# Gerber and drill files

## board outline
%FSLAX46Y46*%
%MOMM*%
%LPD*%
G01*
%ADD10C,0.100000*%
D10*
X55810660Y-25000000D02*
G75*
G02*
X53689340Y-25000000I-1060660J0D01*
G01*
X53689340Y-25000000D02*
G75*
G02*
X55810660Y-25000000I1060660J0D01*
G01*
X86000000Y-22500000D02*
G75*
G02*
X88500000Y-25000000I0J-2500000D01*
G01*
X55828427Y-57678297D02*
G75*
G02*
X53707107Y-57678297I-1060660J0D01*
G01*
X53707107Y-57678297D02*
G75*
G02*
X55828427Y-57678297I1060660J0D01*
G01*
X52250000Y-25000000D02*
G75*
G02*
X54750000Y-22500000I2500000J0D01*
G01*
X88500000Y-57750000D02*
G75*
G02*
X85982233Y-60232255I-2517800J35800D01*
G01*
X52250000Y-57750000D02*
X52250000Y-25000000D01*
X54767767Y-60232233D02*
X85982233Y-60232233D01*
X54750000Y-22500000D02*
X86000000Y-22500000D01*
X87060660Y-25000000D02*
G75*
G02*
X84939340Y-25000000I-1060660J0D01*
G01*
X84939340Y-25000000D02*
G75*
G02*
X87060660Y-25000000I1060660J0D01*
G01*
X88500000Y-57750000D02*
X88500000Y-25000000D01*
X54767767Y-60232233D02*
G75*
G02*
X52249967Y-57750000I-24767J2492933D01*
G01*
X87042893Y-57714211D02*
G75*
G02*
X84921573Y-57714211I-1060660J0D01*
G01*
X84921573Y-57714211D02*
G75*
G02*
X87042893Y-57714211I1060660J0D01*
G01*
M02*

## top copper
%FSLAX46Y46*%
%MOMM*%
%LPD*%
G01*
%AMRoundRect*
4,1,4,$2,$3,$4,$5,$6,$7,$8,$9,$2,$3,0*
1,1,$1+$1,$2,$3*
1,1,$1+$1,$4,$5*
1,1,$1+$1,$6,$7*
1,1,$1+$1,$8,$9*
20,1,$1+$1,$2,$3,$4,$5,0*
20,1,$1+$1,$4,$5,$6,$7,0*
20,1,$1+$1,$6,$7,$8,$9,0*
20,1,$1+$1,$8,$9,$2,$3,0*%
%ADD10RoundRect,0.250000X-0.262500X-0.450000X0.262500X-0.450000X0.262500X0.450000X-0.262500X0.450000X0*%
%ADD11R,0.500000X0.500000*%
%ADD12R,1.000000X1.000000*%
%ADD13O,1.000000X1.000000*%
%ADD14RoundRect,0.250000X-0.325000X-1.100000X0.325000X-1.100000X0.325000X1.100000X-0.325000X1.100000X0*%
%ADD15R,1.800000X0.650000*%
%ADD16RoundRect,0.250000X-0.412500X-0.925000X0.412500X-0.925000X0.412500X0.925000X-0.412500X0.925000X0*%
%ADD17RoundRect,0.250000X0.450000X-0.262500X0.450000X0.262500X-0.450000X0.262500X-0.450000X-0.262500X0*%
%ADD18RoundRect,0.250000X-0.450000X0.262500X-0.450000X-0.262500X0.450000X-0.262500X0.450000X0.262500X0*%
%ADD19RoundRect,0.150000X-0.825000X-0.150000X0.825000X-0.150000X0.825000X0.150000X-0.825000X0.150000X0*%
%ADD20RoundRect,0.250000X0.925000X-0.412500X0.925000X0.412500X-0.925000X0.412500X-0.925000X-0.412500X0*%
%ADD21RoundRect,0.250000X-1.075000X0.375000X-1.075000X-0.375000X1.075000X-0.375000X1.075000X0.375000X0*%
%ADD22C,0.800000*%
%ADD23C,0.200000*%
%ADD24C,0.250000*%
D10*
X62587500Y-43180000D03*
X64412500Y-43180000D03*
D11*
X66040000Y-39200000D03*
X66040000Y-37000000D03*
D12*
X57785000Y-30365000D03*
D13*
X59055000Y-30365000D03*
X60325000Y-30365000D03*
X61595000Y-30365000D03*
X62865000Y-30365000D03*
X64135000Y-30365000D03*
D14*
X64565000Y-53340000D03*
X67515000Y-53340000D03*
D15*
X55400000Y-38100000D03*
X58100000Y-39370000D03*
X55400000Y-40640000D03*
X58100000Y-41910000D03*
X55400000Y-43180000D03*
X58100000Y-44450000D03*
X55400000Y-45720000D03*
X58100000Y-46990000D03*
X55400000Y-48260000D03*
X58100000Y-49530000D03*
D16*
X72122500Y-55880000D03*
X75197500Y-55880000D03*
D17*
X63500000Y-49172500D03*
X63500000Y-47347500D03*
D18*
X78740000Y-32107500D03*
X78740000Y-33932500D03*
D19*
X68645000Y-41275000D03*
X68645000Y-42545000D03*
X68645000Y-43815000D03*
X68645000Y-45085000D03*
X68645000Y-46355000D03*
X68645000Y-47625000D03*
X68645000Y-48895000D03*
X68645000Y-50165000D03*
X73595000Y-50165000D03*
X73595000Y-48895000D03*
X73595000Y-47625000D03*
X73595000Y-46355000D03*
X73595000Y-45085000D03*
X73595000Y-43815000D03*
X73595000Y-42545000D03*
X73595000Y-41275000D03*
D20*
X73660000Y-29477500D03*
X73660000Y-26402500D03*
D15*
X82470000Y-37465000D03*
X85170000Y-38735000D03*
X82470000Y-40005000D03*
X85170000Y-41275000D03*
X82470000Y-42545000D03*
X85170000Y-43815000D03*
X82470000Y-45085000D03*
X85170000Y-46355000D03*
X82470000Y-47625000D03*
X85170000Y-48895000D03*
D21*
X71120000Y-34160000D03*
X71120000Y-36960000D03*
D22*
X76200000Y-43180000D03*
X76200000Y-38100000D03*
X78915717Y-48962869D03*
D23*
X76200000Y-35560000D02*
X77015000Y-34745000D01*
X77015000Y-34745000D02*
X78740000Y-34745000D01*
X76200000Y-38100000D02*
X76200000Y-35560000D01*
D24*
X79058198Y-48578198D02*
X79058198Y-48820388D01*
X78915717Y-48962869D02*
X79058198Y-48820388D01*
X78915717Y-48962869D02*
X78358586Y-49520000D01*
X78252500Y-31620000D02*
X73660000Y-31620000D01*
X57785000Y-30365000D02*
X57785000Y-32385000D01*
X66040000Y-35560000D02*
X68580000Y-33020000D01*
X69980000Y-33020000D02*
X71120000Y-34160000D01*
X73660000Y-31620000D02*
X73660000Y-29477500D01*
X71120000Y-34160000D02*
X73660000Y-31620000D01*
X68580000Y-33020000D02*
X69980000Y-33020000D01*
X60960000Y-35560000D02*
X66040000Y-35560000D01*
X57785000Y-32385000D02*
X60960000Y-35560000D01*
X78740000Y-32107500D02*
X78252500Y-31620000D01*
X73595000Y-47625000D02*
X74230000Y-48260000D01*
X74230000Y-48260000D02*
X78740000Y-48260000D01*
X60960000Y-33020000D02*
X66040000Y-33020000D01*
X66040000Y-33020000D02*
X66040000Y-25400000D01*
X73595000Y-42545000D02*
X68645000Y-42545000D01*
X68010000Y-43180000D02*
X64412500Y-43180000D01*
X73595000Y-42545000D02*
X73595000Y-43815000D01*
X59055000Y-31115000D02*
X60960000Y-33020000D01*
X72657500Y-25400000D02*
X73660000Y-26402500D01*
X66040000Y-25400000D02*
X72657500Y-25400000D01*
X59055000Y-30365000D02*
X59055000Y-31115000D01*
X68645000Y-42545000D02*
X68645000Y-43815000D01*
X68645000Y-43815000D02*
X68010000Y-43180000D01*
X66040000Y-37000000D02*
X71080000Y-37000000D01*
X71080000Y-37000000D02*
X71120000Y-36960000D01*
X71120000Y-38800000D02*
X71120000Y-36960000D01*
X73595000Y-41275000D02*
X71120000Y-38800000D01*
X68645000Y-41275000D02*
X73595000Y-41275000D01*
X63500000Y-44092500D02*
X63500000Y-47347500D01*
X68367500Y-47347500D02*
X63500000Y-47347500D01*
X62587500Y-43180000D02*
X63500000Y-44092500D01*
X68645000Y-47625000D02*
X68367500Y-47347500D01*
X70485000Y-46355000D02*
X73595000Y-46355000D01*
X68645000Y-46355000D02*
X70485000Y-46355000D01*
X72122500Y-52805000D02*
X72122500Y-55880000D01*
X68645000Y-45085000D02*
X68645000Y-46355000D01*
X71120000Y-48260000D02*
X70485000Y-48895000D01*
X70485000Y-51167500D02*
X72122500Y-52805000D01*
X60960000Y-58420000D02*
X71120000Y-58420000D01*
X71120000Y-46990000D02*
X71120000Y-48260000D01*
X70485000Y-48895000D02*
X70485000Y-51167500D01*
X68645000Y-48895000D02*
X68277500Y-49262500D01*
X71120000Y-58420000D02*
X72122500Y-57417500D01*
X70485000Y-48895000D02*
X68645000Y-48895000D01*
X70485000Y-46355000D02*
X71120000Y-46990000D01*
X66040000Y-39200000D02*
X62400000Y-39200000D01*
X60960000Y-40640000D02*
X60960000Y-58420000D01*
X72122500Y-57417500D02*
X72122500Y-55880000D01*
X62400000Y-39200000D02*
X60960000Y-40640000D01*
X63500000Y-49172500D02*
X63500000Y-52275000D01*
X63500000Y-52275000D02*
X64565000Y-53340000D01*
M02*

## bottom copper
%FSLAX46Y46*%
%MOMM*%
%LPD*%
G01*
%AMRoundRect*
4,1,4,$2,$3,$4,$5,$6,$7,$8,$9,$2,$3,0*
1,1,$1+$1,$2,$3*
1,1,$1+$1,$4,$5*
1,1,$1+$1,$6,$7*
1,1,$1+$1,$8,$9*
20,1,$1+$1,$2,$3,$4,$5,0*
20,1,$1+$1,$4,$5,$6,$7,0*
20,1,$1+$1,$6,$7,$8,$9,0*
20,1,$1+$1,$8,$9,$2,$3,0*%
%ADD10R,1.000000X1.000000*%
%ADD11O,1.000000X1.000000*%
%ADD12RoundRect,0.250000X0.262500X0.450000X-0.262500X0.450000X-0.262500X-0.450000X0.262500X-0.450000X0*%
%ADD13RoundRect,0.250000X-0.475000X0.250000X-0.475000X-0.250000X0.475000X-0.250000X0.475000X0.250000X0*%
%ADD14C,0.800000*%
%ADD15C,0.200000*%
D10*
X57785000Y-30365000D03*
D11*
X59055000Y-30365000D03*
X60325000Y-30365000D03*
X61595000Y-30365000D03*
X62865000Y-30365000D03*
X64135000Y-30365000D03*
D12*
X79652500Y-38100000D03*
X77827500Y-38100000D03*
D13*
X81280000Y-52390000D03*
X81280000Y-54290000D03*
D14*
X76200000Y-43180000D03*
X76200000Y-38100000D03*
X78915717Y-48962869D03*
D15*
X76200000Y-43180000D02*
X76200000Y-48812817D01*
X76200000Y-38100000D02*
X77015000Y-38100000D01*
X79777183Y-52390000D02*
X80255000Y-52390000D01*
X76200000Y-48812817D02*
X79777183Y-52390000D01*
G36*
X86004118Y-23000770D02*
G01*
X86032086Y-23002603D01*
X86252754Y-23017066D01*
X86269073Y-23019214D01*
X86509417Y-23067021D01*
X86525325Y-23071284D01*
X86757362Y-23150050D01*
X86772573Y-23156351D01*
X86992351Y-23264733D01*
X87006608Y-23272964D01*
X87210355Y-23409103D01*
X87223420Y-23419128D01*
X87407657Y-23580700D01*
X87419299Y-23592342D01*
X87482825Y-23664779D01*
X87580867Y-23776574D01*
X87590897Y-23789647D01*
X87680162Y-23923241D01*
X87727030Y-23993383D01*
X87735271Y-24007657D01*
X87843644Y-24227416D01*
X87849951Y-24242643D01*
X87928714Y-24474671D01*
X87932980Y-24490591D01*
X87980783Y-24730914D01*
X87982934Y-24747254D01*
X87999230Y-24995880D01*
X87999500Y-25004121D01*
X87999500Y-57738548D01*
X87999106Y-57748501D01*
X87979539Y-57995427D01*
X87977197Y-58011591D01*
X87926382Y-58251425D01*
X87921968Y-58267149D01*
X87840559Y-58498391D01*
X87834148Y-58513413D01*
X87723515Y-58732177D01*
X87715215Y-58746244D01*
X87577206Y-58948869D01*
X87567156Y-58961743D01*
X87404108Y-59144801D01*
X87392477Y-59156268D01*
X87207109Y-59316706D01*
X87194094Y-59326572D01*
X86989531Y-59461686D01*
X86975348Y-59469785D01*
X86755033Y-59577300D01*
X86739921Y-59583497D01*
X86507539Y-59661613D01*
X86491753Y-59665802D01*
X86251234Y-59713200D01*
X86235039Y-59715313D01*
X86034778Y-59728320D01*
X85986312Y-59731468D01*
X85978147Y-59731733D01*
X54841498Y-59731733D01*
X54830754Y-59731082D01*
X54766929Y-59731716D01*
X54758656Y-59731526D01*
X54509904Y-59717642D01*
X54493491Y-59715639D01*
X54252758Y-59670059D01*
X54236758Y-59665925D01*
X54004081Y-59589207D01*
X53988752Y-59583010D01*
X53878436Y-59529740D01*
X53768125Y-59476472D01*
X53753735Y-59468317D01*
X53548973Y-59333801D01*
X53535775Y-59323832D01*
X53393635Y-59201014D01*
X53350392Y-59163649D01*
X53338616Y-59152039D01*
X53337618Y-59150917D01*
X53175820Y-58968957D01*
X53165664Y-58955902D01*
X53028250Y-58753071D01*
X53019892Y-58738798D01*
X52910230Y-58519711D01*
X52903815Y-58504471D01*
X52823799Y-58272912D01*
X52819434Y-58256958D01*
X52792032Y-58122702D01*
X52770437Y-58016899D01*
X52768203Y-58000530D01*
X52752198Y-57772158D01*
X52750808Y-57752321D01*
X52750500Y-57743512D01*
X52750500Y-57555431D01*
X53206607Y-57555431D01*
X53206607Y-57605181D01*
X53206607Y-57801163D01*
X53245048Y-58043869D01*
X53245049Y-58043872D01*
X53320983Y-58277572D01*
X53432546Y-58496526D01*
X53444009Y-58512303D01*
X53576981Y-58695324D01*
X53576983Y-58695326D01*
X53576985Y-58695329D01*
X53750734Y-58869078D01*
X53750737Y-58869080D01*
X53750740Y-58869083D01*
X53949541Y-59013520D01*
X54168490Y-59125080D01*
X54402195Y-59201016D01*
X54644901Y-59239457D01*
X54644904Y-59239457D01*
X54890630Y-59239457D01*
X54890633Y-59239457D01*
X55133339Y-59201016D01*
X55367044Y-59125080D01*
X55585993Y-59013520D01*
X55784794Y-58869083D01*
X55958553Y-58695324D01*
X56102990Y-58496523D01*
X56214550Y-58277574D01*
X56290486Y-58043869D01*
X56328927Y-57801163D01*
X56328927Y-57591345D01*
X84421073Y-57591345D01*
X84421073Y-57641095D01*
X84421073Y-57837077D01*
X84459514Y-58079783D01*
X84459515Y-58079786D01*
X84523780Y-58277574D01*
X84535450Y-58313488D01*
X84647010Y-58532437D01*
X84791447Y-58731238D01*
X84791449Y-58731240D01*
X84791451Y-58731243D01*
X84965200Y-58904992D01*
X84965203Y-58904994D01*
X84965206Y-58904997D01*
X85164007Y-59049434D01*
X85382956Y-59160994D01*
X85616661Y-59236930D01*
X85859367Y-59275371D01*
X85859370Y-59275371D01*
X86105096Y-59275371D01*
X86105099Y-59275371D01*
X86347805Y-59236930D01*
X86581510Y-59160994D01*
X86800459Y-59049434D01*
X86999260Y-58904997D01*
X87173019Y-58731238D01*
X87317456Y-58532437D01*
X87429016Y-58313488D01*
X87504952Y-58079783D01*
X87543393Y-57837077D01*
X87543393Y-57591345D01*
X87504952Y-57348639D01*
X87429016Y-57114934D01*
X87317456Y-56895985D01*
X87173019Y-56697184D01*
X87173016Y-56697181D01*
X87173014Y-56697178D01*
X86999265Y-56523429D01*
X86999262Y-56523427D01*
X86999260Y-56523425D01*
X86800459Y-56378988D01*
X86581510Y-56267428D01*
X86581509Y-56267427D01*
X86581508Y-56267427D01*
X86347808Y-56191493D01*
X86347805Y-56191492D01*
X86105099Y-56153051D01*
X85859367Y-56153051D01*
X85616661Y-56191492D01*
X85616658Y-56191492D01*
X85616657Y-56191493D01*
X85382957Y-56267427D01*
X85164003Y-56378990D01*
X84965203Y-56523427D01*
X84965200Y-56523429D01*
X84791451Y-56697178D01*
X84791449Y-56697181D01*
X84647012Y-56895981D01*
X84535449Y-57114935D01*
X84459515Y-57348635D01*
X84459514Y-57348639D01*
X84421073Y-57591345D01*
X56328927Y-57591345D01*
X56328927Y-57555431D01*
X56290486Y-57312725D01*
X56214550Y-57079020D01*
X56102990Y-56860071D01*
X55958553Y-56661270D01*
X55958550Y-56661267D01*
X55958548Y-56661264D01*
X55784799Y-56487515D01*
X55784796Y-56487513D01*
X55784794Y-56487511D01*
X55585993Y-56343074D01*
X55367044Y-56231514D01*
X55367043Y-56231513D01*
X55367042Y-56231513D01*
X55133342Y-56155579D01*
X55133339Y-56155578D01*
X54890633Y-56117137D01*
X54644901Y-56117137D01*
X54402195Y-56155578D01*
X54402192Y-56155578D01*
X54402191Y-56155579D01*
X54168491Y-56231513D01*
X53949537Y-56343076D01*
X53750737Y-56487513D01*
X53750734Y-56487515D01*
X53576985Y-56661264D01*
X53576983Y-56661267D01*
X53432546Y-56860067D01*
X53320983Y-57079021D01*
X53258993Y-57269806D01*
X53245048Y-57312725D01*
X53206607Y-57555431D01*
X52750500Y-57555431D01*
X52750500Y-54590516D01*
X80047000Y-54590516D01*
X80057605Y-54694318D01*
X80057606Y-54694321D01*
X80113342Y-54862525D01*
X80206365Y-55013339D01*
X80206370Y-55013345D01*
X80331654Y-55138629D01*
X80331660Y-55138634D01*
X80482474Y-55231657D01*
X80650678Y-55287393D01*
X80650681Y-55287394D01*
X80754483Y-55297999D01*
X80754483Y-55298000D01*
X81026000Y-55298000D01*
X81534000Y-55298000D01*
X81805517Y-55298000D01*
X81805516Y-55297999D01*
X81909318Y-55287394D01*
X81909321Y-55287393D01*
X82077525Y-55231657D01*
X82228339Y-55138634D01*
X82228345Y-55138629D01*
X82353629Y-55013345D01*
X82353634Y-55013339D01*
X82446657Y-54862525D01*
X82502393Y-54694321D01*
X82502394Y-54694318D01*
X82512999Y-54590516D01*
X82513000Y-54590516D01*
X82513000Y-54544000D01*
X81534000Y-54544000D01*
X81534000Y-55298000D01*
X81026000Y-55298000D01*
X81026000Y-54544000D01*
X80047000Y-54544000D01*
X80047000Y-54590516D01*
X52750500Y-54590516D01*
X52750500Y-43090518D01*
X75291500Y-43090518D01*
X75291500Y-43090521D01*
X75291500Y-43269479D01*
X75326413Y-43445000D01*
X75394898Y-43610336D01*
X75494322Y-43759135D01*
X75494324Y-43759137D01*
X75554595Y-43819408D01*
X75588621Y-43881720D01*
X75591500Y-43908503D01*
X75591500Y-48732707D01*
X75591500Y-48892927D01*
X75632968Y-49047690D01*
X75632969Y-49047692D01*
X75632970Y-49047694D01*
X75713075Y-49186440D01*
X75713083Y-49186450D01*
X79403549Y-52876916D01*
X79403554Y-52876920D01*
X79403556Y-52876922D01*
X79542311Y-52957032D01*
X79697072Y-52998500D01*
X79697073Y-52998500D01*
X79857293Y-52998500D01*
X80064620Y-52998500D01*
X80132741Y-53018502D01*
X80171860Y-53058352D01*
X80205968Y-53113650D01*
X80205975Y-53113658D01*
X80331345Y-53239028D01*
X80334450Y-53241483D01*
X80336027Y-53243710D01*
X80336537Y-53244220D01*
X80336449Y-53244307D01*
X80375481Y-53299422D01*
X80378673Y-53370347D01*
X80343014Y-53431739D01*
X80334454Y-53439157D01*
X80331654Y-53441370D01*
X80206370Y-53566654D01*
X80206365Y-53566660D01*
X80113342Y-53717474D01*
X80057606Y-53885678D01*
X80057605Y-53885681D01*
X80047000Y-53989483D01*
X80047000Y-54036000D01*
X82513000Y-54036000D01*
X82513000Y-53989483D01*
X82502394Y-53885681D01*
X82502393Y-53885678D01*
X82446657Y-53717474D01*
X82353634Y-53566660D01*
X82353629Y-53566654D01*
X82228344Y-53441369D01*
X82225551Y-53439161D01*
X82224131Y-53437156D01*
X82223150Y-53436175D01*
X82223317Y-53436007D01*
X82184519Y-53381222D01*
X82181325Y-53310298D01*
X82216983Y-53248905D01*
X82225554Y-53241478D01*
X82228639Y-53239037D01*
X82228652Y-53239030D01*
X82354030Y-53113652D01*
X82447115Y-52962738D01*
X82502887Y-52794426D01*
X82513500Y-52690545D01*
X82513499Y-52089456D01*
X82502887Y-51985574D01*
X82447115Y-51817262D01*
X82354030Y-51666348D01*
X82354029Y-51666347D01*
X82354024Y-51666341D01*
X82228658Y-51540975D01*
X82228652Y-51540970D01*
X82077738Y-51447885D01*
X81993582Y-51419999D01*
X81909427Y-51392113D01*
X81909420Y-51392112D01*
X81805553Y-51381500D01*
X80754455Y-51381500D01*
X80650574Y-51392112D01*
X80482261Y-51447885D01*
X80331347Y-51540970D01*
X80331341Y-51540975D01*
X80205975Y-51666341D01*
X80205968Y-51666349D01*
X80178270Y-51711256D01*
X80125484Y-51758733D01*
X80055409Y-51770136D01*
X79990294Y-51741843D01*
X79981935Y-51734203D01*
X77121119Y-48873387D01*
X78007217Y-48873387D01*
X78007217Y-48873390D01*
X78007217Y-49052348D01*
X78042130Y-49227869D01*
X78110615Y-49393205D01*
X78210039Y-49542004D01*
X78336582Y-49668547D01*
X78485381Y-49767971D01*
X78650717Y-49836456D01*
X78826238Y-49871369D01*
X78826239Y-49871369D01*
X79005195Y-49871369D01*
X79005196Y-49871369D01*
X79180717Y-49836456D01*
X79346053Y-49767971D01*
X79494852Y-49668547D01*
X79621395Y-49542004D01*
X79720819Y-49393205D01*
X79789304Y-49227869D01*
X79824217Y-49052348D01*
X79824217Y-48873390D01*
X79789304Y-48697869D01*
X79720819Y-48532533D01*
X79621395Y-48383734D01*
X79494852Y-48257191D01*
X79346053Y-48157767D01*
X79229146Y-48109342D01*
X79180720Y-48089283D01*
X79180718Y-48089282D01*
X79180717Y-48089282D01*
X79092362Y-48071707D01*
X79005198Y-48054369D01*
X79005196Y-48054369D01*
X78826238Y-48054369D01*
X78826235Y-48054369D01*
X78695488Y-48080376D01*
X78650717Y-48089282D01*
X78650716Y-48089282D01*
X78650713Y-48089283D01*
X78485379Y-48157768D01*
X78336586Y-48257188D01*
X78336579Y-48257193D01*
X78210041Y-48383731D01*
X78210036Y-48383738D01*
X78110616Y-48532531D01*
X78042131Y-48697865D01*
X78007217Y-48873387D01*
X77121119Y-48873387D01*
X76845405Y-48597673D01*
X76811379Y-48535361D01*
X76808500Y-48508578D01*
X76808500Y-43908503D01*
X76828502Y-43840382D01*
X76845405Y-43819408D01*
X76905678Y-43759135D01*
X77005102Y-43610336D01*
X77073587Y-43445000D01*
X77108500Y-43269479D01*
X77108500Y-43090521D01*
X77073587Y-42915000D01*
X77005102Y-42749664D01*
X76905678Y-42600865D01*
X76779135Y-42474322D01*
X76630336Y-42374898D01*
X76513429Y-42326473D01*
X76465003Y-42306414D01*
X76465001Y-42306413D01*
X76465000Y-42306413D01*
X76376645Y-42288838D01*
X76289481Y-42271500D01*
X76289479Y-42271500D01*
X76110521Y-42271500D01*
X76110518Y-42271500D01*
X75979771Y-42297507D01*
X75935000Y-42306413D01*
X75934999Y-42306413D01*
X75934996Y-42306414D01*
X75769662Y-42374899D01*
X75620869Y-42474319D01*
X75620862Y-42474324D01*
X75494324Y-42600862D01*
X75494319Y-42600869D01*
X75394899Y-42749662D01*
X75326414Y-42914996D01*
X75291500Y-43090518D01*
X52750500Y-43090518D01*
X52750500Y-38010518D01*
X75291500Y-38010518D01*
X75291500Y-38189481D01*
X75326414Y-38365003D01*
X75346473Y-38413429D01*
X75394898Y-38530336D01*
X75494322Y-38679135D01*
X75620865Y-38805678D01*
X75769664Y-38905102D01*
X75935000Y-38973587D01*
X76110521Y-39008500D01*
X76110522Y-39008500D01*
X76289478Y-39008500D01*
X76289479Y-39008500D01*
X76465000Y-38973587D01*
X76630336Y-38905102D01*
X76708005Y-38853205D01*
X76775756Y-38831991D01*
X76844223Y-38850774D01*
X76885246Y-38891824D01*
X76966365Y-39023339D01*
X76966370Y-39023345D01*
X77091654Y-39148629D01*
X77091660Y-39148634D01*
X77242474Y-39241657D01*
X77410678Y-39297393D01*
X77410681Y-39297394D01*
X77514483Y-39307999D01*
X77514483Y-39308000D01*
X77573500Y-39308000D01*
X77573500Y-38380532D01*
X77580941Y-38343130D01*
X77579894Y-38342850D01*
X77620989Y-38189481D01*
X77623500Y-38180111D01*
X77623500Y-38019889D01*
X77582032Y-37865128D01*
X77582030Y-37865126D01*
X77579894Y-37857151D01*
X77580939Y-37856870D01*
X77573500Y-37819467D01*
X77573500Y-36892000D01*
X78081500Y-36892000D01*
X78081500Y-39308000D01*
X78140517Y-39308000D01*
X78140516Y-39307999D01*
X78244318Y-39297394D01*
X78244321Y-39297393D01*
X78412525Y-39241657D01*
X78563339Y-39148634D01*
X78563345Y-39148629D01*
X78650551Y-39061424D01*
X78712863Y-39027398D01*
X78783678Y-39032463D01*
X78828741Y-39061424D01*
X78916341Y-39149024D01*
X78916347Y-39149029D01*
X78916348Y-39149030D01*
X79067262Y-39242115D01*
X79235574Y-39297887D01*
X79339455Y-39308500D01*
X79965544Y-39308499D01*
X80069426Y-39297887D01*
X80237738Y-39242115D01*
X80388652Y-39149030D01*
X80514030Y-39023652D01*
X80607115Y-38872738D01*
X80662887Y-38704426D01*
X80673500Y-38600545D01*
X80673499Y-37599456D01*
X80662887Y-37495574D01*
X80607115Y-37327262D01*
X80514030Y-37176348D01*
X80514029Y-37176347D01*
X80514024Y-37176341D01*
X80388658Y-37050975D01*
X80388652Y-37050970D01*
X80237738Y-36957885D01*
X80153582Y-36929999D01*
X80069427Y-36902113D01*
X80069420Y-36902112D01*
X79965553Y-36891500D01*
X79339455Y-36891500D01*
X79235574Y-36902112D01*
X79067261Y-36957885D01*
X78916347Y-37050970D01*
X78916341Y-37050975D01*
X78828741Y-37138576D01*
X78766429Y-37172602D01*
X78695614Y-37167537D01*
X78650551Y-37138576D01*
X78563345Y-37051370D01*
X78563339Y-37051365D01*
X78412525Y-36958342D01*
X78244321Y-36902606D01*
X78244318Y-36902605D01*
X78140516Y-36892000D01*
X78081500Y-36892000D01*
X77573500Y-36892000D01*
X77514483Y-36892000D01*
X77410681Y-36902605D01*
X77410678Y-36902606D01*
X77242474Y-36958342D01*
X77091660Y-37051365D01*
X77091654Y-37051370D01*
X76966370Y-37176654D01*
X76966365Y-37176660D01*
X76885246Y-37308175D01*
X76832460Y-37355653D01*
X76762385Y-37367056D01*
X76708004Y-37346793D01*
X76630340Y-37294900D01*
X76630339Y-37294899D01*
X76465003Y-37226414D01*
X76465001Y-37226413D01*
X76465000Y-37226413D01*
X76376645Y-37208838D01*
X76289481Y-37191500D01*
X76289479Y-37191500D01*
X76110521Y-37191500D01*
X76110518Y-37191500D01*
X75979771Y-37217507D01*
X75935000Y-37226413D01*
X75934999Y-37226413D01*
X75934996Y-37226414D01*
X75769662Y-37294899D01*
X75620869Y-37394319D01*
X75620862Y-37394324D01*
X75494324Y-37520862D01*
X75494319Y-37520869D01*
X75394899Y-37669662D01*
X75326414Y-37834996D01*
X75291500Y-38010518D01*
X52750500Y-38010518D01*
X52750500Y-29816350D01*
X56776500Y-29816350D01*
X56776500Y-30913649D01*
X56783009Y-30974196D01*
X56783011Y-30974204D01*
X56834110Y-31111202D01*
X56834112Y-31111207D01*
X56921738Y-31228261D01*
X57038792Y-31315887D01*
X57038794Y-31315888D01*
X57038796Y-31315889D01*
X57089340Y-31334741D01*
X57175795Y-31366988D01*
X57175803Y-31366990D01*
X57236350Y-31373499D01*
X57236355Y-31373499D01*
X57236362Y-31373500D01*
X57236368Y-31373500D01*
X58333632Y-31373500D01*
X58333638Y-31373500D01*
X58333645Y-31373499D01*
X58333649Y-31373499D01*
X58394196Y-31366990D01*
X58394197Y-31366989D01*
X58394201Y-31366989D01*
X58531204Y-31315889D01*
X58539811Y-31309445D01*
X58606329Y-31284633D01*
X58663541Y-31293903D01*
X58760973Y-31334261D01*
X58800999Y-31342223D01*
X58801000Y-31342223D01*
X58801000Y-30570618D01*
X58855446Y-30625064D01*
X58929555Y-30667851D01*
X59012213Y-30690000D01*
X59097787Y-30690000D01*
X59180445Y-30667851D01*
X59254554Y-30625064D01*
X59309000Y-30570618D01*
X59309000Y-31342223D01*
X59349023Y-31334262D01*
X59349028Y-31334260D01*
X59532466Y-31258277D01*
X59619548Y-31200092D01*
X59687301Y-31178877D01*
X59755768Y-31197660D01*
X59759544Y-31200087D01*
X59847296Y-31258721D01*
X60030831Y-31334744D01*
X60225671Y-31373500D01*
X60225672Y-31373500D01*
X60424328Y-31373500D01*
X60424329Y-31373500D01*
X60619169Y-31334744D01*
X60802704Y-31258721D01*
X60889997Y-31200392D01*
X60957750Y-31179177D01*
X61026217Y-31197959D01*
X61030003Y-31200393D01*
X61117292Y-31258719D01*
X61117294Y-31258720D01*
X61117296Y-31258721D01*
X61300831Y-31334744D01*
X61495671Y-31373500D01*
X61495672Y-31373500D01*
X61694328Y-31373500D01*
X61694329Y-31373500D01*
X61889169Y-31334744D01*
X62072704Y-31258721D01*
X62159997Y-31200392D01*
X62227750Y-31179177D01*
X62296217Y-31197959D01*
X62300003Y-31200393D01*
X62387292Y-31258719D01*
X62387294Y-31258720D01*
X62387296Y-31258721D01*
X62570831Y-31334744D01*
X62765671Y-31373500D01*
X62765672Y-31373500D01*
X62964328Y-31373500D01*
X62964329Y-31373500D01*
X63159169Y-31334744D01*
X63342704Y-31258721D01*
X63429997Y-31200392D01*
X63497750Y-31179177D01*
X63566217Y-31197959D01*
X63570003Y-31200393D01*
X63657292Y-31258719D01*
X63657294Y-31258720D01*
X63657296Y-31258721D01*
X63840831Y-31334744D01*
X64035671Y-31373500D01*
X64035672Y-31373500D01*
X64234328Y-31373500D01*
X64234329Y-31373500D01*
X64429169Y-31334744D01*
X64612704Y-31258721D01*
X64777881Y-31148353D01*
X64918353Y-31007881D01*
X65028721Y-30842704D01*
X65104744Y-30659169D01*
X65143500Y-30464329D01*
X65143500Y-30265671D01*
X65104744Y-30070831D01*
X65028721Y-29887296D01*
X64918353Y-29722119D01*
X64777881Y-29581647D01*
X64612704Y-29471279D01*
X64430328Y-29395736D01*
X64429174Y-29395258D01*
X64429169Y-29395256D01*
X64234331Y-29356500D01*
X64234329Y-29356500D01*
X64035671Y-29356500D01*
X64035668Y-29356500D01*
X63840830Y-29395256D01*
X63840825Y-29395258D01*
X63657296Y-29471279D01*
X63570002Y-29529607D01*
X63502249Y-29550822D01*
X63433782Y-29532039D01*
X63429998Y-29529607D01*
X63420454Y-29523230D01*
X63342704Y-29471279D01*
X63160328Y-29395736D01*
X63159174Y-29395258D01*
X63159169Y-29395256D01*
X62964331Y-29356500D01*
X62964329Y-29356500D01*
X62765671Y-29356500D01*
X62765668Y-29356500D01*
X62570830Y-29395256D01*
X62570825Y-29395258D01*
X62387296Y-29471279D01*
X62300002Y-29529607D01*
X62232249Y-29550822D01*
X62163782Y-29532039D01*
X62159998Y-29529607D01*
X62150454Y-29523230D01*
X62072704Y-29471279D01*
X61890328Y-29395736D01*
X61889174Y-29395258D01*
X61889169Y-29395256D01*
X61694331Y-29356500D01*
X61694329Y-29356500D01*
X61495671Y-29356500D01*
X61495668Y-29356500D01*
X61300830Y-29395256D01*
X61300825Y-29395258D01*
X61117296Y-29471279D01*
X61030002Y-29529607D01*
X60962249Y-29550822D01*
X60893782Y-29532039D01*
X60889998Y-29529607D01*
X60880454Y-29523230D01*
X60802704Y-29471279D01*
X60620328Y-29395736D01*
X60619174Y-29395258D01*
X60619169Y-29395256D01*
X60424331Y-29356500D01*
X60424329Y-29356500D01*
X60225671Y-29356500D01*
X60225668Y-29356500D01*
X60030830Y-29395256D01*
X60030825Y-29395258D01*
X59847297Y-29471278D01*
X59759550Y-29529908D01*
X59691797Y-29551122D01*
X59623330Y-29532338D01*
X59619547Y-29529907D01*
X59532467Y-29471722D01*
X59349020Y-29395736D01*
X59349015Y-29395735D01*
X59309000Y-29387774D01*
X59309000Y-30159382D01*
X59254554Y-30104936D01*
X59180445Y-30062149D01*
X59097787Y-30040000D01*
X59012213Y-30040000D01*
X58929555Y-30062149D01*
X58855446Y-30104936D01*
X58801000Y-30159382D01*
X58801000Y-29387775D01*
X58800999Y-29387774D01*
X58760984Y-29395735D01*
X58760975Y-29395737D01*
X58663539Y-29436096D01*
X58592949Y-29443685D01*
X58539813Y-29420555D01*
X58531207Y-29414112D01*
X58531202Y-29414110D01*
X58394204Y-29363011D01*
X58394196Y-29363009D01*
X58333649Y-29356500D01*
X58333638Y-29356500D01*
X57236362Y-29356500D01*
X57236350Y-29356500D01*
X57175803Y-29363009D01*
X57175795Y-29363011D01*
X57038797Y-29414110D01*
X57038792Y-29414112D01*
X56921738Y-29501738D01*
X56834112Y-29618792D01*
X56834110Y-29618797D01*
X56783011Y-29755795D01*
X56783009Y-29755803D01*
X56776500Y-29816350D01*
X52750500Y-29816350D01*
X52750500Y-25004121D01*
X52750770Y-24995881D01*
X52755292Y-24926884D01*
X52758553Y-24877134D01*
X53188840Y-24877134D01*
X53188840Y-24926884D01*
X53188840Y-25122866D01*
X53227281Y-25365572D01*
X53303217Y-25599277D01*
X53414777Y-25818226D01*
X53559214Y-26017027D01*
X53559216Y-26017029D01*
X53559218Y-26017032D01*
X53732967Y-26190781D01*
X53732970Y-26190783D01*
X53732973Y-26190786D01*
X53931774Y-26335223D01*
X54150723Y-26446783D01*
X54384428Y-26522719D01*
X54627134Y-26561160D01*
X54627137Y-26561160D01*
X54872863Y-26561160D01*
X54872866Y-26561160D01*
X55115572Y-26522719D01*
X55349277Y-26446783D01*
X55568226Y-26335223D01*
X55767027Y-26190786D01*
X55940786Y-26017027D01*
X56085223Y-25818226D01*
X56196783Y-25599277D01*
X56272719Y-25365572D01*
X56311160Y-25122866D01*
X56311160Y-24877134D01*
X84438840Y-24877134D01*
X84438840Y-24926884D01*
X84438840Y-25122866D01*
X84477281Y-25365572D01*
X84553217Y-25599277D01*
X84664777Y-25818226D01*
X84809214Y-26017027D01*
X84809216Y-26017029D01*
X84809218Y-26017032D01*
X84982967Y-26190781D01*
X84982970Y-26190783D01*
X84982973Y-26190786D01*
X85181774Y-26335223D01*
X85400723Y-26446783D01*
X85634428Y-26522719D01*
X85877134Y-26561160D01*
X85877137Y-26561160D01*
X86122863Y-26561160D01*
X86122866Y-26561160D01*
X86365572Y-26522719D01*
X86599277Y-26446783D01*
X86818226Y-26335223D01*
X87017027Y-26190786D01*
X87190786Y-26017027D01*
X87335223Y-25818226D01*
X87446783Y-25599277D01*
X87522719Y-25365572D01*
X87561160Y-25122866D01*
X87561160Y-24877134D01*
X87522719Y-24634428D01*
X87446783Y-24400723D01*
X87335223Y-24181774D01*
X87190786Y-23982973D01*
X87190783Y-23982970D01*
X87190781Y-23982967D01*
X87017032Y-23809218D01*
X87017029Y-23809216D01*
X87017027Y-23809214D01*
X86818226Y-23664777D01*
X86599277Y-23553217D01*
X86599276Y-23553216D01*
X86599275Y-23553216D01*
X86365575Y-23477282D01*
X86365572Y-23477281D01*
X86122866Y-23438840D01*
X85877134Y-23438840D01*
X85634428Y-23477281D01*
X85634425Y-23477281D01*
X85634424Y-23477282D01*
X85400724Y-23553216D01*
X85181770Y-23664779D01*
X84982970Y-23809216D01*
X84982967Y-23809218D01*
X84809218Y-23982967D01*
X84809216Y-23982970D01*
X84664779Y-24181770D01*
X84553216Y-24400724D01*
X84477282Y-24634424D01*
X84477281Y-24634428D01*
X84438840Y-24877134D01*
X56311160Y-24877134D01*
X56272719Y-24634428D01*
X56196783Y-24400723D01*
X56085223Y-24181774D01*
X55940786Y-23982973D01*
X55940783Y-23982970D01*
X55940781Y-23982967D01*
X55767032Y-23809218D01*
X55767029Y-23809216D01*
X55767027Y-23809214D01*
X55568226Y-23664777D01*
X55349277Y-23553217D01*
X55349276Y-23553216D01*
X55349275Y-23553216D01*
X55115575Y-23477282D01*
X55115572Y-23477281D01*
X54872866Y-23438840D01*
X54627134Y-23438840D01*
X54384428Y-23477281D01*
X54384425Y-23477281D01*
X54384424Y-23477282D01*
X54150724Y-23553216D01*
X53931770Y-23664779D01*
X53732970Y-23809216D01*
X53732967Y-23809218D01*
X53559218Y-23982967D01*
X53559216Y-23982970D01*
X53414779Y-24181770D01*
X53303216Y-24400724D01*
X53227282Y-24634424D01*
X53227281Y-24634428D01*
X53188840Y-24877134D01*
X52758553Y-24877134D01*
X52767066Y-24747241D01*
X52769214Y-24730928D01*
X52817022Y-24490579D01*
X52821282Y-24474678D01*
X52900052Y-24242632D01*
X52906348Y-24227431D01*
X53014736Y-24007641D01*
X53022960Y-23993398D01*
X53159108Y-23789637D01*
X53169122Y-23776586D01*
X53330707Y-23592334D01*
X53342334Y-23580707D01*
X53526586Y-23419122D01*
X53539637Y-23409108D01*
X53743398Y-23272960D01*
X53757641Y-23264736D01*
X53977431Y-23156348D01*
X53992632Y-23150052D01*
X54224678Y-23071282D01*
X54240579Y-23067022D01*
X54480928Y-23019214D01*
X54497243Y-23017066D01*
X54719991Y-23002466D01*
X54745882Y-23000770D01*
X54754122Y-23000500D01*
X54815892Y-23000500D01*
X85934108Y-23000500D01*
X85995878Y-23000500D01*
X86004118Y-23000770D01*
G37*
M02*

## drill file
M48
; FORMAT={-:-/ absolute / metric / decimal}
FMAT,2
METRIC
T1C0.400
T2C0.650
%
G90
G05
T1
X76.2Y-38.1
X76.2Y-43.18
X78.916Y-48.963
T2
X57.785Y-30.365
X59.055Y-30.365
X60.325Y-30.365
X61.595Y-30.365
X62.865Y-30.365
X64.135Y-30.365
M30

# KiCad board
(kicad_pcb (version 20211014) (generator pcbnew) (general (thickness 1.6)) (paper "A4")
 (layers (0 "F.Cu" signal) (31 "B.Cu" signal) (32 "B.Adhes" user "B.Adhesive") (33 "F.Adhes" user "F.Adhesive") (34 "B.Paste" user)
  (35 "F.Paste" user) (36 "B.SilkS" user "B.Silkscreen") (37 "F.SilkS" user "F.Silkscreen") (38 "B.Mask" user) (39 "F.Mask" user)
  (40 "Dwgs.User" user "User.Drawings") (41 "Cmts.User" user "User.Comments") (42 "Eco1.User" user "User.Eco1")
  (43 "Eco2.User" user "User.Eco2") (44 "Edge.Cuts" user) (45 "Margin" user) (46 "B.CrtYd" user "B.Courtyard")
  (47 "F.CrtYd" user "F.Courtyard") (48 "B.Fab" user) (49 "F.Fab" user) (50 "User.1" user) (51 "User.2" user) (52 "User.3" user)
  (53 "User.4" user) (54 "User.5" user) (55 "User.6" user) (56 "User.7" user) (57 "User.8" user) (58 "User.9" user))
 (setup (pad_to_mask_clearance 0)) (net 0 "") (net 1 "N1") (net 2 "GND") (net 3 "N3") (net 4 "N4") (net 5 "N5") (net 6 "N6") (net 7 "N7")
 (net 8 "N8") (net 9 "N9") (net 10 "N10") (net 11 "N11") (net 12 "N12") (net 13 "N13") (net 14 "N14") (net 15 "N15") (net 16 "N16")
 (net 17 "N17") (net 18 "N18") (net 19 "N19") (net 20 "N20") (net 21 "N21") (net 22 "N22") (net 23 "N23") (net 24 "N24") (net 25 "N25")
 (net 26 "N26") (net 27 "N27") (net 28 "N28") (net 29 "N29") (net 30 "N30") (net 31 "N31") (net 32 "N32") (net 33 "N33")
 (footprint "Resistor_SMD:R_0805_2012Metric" (layer "F.Cu") (at 63.5 43.18)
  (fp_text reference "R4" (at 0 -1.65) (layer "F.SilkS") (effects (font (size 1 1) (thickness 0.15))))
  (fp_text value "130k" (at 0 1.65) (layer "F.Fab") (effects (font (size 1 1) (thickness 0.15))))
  (pad "1" smd roundrect (at -0.9125 0) (size 1.025 1.4) (layers "F.Cu" "F.Paste" "F.Mask") (roundrect_rratio 0.243902) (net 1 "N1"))
  (pad "2" smd roundrect (at 0.9125 0) (size 1.025 1.4) (layers "F.Cu" "F.Paste" "F.Mask") (roundrect_rratio 0.243902) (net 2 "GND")))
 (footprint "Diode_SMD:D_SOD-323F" (layer "F.Cu") (at 66.04 38.1 90)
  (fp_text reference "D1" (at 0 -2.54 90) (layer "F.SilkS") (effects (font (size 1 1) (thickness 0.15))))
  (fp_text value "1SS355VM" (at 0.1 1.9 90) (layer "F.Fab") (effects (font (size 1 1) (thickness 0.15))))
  (pad "1" smd rect (at -1.1 0 90) (size 0.5 0.5) (layers "F.Cu" "F.Paste" "F.Mask") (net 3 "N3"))
  (pad "2" smd rect (at 1.1 0 90) (size 0.5 0.5) (layers "F.Cu" "F.Paste" "F.Mask") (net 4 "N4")))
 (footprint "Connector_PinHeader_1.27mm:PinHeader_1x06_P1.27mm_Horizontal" (layer "F.Cu") (at 57.785 30.365 90)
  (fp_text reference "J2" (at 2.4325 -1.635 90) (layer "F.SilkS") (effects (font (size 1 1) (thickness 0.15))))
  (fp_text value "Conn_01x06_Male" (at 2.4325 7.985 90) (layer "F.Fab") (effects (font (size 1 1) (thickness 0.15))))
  (pad "1" thru_hole rect (at 0 0 90) (size 1 1) (drill 0.65) (layers *.Cu *.Mask) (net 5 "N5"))
  (pad "2" thru_hole oval (at 0 1.27 90) (size 1 1) (drill 0.65) (layers *.Cu *.Mask) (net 2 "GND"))
  (pad "3" thru_hole oval (at 0 2.54 90) (size 1 1) (drill 0.65) (layers *.Cu *.Mask) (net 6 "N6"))
  (pad "4" thru_hole oval (at 0 3.81 90) (size 1 1) (drill 0.65) (layers *.Cu *.Mask) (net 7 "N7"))
  (pad "5" thru_hole oval (at 0 5.08 90) (size 1 1) (drill 0.65) (layers *.Cu *.Mask) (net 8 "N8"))
  (pad "6" thru_hole oval (at 0 6.35 90) (size 1 1) (drill 0.65) (layers *.Cu *.Mask) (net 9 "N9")))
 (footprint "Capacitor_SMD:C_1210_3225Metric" (layer "F.Cu") (at 66.04 53.34)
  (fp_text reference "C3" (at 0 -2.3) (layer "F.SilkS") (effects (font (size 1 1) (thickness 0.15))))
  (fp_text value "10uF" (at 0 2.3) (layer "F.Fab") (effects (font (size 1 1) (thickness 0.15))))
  (pad "1" smd roundrect (at -1.475 0) (size 1.15 2.7) (layers "F.Cu" "F.Paste" "F.Mask") (roundrect_rratio 0.217391) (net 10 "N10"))
  (pad "2" smd roundrect (at 1.475 0) (size 1.15 2.7) (layers "F.Cu" "F.Paste" "F.Mask") (roundrect_rratio 0.217391) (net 2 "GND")))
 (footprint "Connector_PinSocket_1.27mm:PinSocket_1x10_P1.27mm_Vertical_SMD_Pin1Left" (layer "F.Cu") (at 56.75 43.815)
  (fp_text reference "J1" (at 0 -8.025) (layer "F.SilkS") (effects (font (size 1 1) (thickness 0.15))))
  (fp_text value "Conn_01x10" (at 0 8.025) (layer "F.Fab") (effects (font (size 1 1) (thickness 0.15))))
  (pad "1" smd rect (at -1.35 -5.715) (size 1.8 0.65) (layers "F.Cu" "F.Paste" "F.Mask") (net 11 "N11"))
  (pad "2" smd rect (at 1.35 -4.445) (size 1.8 0.65) (layers "F.Cu" "F.Paste" "F.Mask") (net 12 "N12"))
  (pad "3" smd rect (at -1.35 -3.175) (size 1.8 0.65) (layers "F.Cu" "F.Paste" "F.Mask") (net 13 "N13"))
  (pad "4" smd rect (at 1.35 -1.905) (size 1.8 0.65) (layers "F.Cu" "F.Paste" "F.Mask") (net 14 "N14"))
  (pad "5" smd rect (at -1.35 -0.635) (size 1.8 0.65) (layers "F.Cu" "F.Paste" "F.Mask") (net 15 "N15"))
  (pad "6" smd rect (at 1.35 0.635) (size 1.8 0.65) (layers "F.Cu" "F.Paste" "F.Mask") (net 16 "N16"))
  (pad "7" smd rect (at -1.35 1.905) (size 1.8 0.65) (layers "F.Cu" "F.Paste" "F.Mask") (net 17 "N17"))
  (pad "8" smd rect (at 1.35 3.175) (size 1.8 0.65) (layers "F.Cu" "F.Paste" "F.Mask") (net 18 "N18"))
  (pad "9" smd rect (at -1.35 4.445) (size 1.8 0.65) (layers "F.Cu" "F.Paste" "F.Mask") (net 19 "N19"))
  (pad "10" smd rect (at 1.35 5.715) (size 1.8 0.65) (layers "F.Cu" "F.Paste" "F.Mask") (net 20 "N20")))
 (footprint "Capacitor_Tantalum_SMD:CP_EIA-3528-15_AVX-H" (layer "F.Cu") (at 73.66 55.88)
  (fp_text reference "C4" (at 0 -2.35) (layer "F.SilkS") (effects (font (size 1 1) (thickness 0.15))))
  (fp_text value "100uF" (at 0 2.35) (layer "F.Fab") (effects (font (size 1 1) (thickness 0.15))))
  (pad "1" smd roundrect (at -1.5375 0) (size 1.325 2.35) (layers "F.Cu" "F.Paste" "F.Mask") (roundrect_rratio 0.188679) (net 3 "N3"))
  (pad "2" smd roundrect (at 1.5375 0) (size 1.325 2.35) (layers "F.Cu" "F.Paste" "F.Mask") (roundrect_rratio 0.188679) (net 2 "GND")))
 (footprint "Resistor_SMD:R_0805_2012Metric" (layer "F.Cu") (at 63.5 48.26 90)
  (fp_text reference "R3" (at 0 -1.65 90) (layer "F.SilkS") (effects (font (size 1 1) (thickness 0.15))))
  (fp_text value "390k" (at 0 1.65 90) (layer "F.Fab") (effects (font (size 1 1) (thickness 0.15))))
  (pad "1" smd roundrect (at -0.9125 0 90) (size 1.025 1.4) (layers "F.Cu" "F.Paste" "F.Mask") (roundrect_rratio 0.243902) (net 10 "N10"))
  (pad "2" smd roundrect (at 0.9125 0 90) (size 1.025 1.4) (layers "F.Cu" "F.Paste" "F.Mask") (roundrect_rratio 0.243902) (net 1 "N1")))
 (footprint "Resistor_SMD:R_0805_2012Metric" (layer "F.Cu") (at 78.74 33.02 -90)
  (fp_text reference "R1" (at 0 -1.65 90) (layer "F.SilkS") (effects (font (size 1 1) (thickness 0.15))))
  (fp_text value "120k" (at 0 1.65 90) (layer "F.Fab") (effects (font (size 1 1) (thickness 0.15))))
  (pad "1" smd roundrect (at -0.9125 0 270) (size 1.025 1.4) (layers "F.Cu" "F.Paste" "F.Mask") (roundrect_rratio 0.243902) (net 5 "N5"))
  (pad "2" smd roundrect (at 0.9125 0 270) (size 1.025 1.4) (layers "F.Cu" "F.Paste" "F.Mask") (roundrect_rratio 0.243902) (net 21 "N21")))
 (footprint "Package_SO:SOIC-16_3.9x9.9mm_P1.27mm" (layer "F.Cu") (at 71.12 45.72)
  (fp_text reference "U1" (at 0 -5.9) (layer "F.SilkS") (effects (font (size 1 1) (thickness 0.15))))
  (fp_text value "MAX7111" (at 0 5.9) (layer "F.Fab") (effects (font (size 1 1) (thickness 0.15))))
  (pad "1" smd roundrect (at -2.475 -4.445) (size 1.95 0.6) (layers "F.Cu" "F.Paste" "F.Mask") (roundrect_rratio 0.25) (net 4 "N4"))
  (pad "2" smd roundrect (at -2.475 -3.175) (size 1.95 0.6) (layers "F.Cu" "F.Paste" "F.Mask") (roundrect_rratio 0.25) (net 2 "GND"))
  (pad "3" smd roundrect (at -2.475 -1.905) (size 1.95 0.6) (layers "F.Cu" "F.Paste" "F.Mask") (roundrect_rratio 0.25) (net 2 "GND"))
  (pad "4" smd roundrect (at -2.475 -0.635) (size 1.95 0.6) (layers "F.Cu" "F.Paste" "F.Mask") (roundrect_rratio 0.25) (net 3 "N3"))
  (pad "5" smd roundrect (at -2.475 0.635) (size 1.95 0.6) (layers "F.Cu" "F.Paste" "F.Mask") (roundrect_rratio 0.25) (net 3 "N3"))
  (pad "6" smd roundrect (at -2.475 1.905) (size 1.95 0.6) (layers "F.Cu" "F.Paste" "F.Mask") (roundrect_rratio 0.25) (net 1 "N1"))
  (pad "7" smd roundrect (at -2.475 3.175) (size 1.95 0.6) (layers "F.Cu" "F.Paste" "F.Mask") (roundrect_rratio 0.25) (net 3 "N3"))
  (pad "8" smd roundrect (at -2.475 4.445) (size 1.95 0.6) (layers "F.Cu" "F.Paste" "F.Mask") (roundrect_rratio 0.25) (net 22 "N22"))
  (pad "9" smd roundrect (at 2.475 4.445) (size 1.95 0.6) (layers "F.Cu" "F.Paste" "F.Mask") (roundrect_rratio 0.25) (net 10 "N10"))
  (pad "10" smd roundrect (at 2.475 3.175) (size 1.95 0.6) (layers "F.Cu" "F.Paste" "F.Mask") (roundrect_rratio 0.25) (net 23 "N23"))
  (pad "11" smd roundrect (at 2.475 1.905) (size 1.95 0.6) (layers "F.Cu" "F.Paste" "F.Mask") (roundrect_rratio 0.25) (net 21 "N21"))
  (pad "12" smd roundrect (at 2.475 0.635) (size 1.95 0.6) (layers "F.Cu" "F.Paste" "F.Mask") (roundrect_rratio 0.25) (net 3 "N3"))
  (pad "13" smd roundrect (at 2.475 -0.635) (size 1.95 0.6) (layers "F.Cu" "F.Paste" "F.Mask") (roundrect_rratio 0.25) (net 23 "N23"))
  (pad "14" smd roundrect (at 2.475 -1.905) (size 1.95 0.6) (layers "F.Cu" "F.Paste" "F.Mask") (roundrect_rratio 0.25) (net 2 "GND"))
  (pad "15" smd roundrect (at 2.475 -3.175) (size 1.95 0.6) (layers "F.Cu" "F.Paste" "F.Mask") (roundrect_rratio 0.25) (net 2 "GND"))
  (pad "16" smd roundrect (at 2.475 -4.445) (size 1.95 0.6) (layers "F.Cu" "F.Paste" "F.Mask") (roundrect_rratio 0.25) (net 4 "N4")))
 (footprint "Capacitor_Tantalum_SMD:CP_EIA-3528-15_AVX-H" (layer "F.Cu") (at 73.66 27.94 90)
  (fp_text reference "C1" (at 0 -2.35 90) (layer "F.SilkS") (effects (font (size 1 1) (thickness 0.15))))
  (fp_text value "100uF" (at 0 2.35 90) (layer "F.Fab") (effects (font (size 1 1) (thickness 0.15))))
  (pad "1" smd roundrect (at -1.5375 0 90) (size 1.325 2.35) (layers "F.Cu" "F.Paste" "F.Mask") (roundrect_rratio 0.188679) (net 5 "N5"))
  (pad "2" smd roundrect (at 1.5375 0 90) (size 1.325 2.35) (layers "F.Cu" "F.Paste" "F.Mask") (roundrect_rratio 0.188679) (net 2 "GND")))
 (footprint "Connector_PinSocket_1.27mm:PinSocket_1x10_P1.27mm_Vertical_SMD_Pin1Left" (layer "F.Cu") (at 83.82 43.18)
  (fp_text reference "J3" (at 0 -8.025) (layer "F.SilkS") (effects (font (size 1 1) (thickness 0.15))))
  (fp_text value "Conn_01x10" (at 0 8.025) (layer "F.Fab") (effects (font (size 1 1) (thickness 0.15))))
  (pad "1" smd rect (at -1.35 -5.715) (size 1.8 0.65) (layers "F.Cu" "F.Paste" "F.Mask") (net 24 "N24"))
  (pad "2" smd rect (at 1.35 -4.445) (size 1.8 0.65) (layers "F.Cu" "F.Paste" "F.Mask") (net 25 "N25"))
  (pad "3" smd rect (at -1.35 -3.175) (size 1.8 0.65) (layers "F.Cu" "F.Paste" "F.Mask") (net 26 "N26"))
  (pad "4" smd rect (at 1.35 -1.905) (size 1.8 0.65) (layers "F.Cu" "F.Paste" "F.Mask") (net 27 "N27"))
  (pad "5" smd rect (at -1.35 -0.635) (size 1.8 0.65) (layers "F.Cu" "F.Paste" "F.Mask") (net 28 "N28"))
  (pad "6" smd rect (at 1.35 0.635) (size 1.8 0.65) (layers "F.Cu" "F.Paste" "F.Mask") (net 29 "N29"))
  (pad "7" smd rect (at -1.35 1.905) (size 1.8 0.65) (layers "F.Cu" "F.Paste" "F.Mask") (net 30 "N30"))
  (pad "8" smd rect (at 1.35 3.175) (size 1.8 0.65) (layers "F.Cu" "F.Paste" "F.Mask") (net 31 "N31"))
  (pad "9" smd rect (at -1.35 4.445) (size 1.8 0.65) (layers "F.Cu" "F.Paste" "F.Mask") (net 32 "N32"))
  (pad "10" smd rect (at 1.35 5.715) (size 1.8 0.65) (layers "F.Cu" "F.Paste" "F.Mask") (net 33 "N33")))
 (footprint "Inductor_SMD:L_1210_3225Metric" (layer "F.Cu") (at 71.12 35.56 -90)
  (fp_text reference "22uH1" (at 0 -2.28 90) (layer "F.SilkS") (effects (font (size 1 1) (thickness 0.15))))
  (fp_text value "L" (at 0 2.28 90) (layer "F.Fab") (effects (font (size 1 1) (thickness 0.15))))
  (pad "1" smd roundrect (at -1.4 0 270) (size 1.25 2.65) (layers "F.Cu" "F.Paste" "F.Mask") (roundrect_rratio 0.2) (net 5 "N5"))
  (pad "2" smd roundrect (at 1.4 0 270) (size 1.25 2.65) (layers "F.Cu" "F.Paste" "F.Mask") (roundrect_rratio 0.2) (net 4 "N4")))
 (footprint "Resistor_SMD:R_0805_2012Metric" (layer "B.Cu") (at 78.74 38.1 180)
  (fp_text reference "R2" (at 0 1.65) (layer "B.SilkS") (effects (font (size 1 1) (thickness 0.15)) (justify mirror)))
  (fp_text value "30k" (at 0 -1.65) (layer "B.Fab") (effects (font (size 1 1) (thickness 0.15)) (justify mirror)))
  (pad "1" smd roundrect (at -0.9125 0 180) (size 1.025 1.4) (layers "B.Cu" "B.Paste" "B.Mask") (roundrect_rratio 0.243902) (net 21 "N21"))
  (pad "2" smd roundrect (at 0.9125 0 180) (size 1.025 1.4) (layers "B.Cu" "B.Paste" "B.Mask") (roundrect_rratio 0.243902) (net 2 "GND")))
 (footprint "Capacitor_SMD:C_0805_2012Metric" (layer "B.Cu") (at 81.28 53.34 -90)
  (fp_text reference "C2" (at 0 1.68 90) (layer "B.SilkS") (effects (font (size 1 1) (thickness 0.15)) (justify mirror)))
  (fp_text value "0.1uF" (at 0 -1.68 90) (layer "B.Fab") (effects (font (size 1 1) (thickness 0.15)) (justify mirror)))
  (pad "1" smd roundrect (at -0.95 0 270) (size 1 1.45) (layers "B.Cu" "B.Paste" "B.Mask") (roundrect_rratio 0.25) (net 23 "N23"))
  (pad "2" smd roundrect (at 0.95 0 270) (size 1 1.45) (layers "B.Cu" "B.Paste" "B.Mask") (roundrect_rratio 0.25) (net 2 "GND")))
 (gr_circle (center 54.75 25) (end 55.5 25.75) (layer "Edge.Cuts") (width 0.1) (fill none))
 (gr_arc (start 86 22.5) (mid 87.767767 23.232233) (end 88.5 25) (layer "Edge.Cuts") (width 0.1))
 (gr_circle (center 54.767767 57.678297) (end 55.517767 58.428297) (layer "Edge.Cuts") (width 0.1) (fill none))
 (gr_arc (start 52.25 25) (mid 52.982233 23.232233) (end 54.75 22.5) (layer "Edge.Cuts") (width 0.1))
 (gr_arc (start 88.5 57.75) (mid 87.750044 59.50733) (end 85.982233 60.232233) (layer "Edge.Cuts") (width 0.1))
 (gr_line (start 52.25 57.75) (end 52.25 25) (layer "Edge.Cuts") (width 0.1))
 (gr_line (start 54.767767 60.232233) (end 85.982233 60.232233) (layer "Edge.Cuts") (width 0.1))
 (gr_line (start 54.75 22.5) (end 86 22.5) (layer "Edge.Cuts") (width 0.1))
 (gr_circle (center 86 25) (end 86.75 25.75) (layer "Edge.Cuts") (width 0.1) (fill none))
 (gr_line (start 88.5 57.75) (end 88.5 25) (layer "Edge.Cuts") (width 0.1))
 (gr_arc (start 54.767767 60.232233) (mid 52.987752 59.509727) (end 52.25 57.75) (layer "Edge.Cuts") (width 0.1))
 (gr_circle (center 85.982233 57.714211) (end 86.732233 58.464211) (layer "Edge.Cuts") (width 0.1) (fill none))
 (segment (start 76.2 35.56) (end 77.015 34.745) (width 0.2) (layer "F.Cu") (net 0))
 (segment (start 77.015 34.745) (end 78.74 34.745) (width 0.2) (layer "F.Cu") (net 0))
 (segment (start 76.2 38.1) (end 76.2 35.56) (width 0.2) (layer "F.Cu") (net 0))
 (segment (start 79.058198 48.578198) (end 79.058198 48.820388) (width 0.25) (layer "F.Cu") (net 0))
 (segment (start 78.915717 48.962869) (end 79.058198 48.820388) (width 0.25) (layer "F.Cu") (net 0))
 (segment (start 78.915717 48.962869) (end 78.358586 49.52) (width 0.25) (layer "F.Cu") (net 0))
 (via (at 76.2 43.18) (size 0.8) (drill 0.4) (layers "F.Cu" "B.Cu") (free) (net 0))
 (via (at 76.2 38.1) (size 0.8) (drill 0.4) (layers "F.Cu" "B.Cu") (free) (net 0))
 (via (at 78.915717 48.962869) (size 0.8) (drill 0.4) (layers "F.Cu" "B.Cu") (free) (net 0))
 (segment (start 76.2 43.18) (end 76.2 48.812817) (width 0.2) (layer "B.Cu") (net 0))
 (segment (start 76.2 38.1) (end 77.015 38.1) (width 0.2) (layer "B.Cu") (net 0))
 (segment (start 79.777183 52.39) (end 80.255 52.39) (width 0.2) (layer "B.Cu") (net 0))
 (segment (start 76.2 48.812817) (end 79.777183 52.39) (width 0.2) (layer "B.Cu") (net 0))
 (segment (start 78.2525 31.62) (end 73.66 31.62) (width 0.25) (layer "F.Cu") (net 5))
 (segment (start 57.785 30.365) (end 57.785 32.385) (width 0.25) (layer "F.Cu") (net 5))
 (segment (start 66.04 35.56) (end 68.58 33.02) (width 0.25) (layer "F.Cu") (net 5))
 (segment (start 69.98 33.02) (end 71.12 34.16) (width 0.25) (layer "F.Cu") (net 5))
 (segment (start 73.66 31.62) (end 73.66 29.4775) (width 0.25) (layer "F.Cu") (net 5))
 (segment (start 71.12 34.16) (end 73.66 31.62) (width 0.25) (layer "F.Cu") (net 5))
 (segment (start 68.58 33.02) (end 69.98 33.02) (width 0.25) (layer "F.Cu") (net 5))
 (segment (start 60.96 35.56) (end 66.04 35.56) (width 0.25) (layer "F.Cu") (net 5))
 (segment (start 57.785 32.385) (end 60.96 35.56) (width 0.25) (layer "F.Cu") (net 5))
 (segment (start 78.74 32.1075) (end 78.2525 31.62) (width 0.25) (layer "F.Cu") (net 5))
 (segment (start 73.595 47.625) (end 74.23 48.26) (width 0.25) (layer "F.Cu") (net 21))
 (segment (start 74.23 48.26) (end 78.74 48.26) (width 0.25) (layer "F.Cu") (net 21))
 (segment (start 60.96 33.02) (end 66.04 33.02) (width 0.25) (layer "F.Cu") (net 2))
 (segment (start 66.04 33.02) (end 66.04 25.4) (width 0.25) (layer "F.Cu") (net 2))
 (segment (start 73.595 42.545) (end 68.645 42.545) (width 0.25) (layer "F.Cu") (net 2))
 (segment (start 68.01 43.18) (end 64.4125 43.18) (width 0.25) (layer "F.Cu") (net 2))
 (segment (start 73.595 42.545) (end 73.595 43.815) (width 0.25) (layer "F.Cu") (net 2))
 (segment (start 59.055 31.115) (end 60.96 33.02) (width 0.25) (layer "F.Cu") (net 2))
 (segment (start 72.6575 25.4) (end 73.66 26.4025) (width 0.25) (layer "F.Cu") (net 2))
 (segment (start 66.04 25.4) (end 72.6575 25.4) (width 0.25) (layer "F.Cu") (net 2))
 (segment (start 59.055 30.365) (end 59.055 31.115) (width 0.25) (layer "F.Cu") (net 2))
 (segment (start 68.645 42.545) (end 68.645 43.815) (width 0.25) (layer "F.Cu") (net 2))
 (segment (start 68.645 43.815) (end 68.01 43.18) (width 0.25) (layer "F.Cu") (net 2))
 (segment (start 66.04 37) (end 71.08 37) (width 0.25) (layer "F.Cu") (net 4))
 (segment (start 71.08 37) (end 71.12 36.96) (width 0.25) (layer "F.Cu") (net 4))
 (segment (start 71.12 38.8) (end 71.12 36.96) (width 0.25) (layer "F.Cu") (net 4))
 (segment (start 73.595 41.275) (end 71.12 38.8) (width 0.25) (layer "F.Cu") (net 4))
 (segment (start 68.645 41.275) (end 73.595 41.275) (width 0.25) (layer "F.Cu") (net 4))
 (segment (start 63.5 44.0925) (end 63.5 47.3475) (width 0.25) (layer "F.Cu") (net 1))
 (segment (start 68.3675 47.3475) (end 63.5 47.3475) (width 0.25) (layer "F.Cu") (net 1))
 (segment (start 62.5875 43.18) (end 63.5 44.0925) (width 0.25) (layer "F.Cu") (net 1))
 (segment (start 68.645 47.625) (end 68.3675 47.3475) (width 0.25) (layer "F.Cu") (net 1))
 (segment (start 70.485 46.355) (end 73.595 46.355) (width 0.25) (layer "F.Cu") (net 3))
 (segment (start 68.645 46.355) (end 70.485 46.355) (width 0.25) (layer "F.Cu") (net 3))
 (segment (start 72.1225 52.805) (end 72.1225 55.88) (width 0.25) (layer "F.Cu") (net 3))
 (segment (start 68.645 45.085) (end 68.645 46.355) (width 0.25) (layer "F.Cu") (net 3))
 (segment (start 71.12 48.26) (end 70.485 48.895) (width 0.25) (layer "F.Cu") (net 3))
 (segment (start 70.485 51.1675) (end 72.1225 52.805) (width 0.25) (layer "F.Cu") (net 3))
 (segment (start 60.96 58.42) (end 71.12 58.42) (width 0.25) (layer "F.Cu") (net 3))
 (segment (start 71.12 46.99) (end 71.12 48.26) (width 0.25) (layer "F.Cu") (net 3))
 (segment (start 70.485 48.895) (end 70.485 51.1675) (width 0.25) (layer "F.Cu") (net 3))
 (segment (start 68.645 48.895) (end 68.2775 49.2625) (width 0.25) (layer "F.Cu") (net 3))
 (segment (start 71.12 58.42) (end 72.1225 57.4175) (width 0.25) (layer "F.Cu") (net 3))
 (segment (start 70.485 48.895) (end 68.645 48.895) (width 0.25) (layer "F.Cu") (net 3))
 (segment (start 70.485 46.355) (end 71.12 46.99) (width 0.25) (layer "F.Cu") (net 3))
 (segment (start 66.04 39.2) (end 62.4 39.2) (width 0.25) (layer "F.Cu") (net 3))
 (segment (start 60.96 40.64) (end 60.96 58.42) (width 0.25) (layer "F.Cu") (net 3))
 (segment (start 72.1225 57.4175) (end 72.1225 55.88) (width 0.25) (layer "F.Cu") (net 3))
 (segment (start 62.4 39.2) (end 60.96 40.64) (width 0.25) (layer "F.Cu") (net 3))
 (segment (start 63.5 49.1725) (end 63.5 52.275) (width 0.25) (layer "F.Cu") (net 10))
 (segment (start 63.5 52.275) (end 64.565 53.34) (width 0.25) (layer "F.Cu") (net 10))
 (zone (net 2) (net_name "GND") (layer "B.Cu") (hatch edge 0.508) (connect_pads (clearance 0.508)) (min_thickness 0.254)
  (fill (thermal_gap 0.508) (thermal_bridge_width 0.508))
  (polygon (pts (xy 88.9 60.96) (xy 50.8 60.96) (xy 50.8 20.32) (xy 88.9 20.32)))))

